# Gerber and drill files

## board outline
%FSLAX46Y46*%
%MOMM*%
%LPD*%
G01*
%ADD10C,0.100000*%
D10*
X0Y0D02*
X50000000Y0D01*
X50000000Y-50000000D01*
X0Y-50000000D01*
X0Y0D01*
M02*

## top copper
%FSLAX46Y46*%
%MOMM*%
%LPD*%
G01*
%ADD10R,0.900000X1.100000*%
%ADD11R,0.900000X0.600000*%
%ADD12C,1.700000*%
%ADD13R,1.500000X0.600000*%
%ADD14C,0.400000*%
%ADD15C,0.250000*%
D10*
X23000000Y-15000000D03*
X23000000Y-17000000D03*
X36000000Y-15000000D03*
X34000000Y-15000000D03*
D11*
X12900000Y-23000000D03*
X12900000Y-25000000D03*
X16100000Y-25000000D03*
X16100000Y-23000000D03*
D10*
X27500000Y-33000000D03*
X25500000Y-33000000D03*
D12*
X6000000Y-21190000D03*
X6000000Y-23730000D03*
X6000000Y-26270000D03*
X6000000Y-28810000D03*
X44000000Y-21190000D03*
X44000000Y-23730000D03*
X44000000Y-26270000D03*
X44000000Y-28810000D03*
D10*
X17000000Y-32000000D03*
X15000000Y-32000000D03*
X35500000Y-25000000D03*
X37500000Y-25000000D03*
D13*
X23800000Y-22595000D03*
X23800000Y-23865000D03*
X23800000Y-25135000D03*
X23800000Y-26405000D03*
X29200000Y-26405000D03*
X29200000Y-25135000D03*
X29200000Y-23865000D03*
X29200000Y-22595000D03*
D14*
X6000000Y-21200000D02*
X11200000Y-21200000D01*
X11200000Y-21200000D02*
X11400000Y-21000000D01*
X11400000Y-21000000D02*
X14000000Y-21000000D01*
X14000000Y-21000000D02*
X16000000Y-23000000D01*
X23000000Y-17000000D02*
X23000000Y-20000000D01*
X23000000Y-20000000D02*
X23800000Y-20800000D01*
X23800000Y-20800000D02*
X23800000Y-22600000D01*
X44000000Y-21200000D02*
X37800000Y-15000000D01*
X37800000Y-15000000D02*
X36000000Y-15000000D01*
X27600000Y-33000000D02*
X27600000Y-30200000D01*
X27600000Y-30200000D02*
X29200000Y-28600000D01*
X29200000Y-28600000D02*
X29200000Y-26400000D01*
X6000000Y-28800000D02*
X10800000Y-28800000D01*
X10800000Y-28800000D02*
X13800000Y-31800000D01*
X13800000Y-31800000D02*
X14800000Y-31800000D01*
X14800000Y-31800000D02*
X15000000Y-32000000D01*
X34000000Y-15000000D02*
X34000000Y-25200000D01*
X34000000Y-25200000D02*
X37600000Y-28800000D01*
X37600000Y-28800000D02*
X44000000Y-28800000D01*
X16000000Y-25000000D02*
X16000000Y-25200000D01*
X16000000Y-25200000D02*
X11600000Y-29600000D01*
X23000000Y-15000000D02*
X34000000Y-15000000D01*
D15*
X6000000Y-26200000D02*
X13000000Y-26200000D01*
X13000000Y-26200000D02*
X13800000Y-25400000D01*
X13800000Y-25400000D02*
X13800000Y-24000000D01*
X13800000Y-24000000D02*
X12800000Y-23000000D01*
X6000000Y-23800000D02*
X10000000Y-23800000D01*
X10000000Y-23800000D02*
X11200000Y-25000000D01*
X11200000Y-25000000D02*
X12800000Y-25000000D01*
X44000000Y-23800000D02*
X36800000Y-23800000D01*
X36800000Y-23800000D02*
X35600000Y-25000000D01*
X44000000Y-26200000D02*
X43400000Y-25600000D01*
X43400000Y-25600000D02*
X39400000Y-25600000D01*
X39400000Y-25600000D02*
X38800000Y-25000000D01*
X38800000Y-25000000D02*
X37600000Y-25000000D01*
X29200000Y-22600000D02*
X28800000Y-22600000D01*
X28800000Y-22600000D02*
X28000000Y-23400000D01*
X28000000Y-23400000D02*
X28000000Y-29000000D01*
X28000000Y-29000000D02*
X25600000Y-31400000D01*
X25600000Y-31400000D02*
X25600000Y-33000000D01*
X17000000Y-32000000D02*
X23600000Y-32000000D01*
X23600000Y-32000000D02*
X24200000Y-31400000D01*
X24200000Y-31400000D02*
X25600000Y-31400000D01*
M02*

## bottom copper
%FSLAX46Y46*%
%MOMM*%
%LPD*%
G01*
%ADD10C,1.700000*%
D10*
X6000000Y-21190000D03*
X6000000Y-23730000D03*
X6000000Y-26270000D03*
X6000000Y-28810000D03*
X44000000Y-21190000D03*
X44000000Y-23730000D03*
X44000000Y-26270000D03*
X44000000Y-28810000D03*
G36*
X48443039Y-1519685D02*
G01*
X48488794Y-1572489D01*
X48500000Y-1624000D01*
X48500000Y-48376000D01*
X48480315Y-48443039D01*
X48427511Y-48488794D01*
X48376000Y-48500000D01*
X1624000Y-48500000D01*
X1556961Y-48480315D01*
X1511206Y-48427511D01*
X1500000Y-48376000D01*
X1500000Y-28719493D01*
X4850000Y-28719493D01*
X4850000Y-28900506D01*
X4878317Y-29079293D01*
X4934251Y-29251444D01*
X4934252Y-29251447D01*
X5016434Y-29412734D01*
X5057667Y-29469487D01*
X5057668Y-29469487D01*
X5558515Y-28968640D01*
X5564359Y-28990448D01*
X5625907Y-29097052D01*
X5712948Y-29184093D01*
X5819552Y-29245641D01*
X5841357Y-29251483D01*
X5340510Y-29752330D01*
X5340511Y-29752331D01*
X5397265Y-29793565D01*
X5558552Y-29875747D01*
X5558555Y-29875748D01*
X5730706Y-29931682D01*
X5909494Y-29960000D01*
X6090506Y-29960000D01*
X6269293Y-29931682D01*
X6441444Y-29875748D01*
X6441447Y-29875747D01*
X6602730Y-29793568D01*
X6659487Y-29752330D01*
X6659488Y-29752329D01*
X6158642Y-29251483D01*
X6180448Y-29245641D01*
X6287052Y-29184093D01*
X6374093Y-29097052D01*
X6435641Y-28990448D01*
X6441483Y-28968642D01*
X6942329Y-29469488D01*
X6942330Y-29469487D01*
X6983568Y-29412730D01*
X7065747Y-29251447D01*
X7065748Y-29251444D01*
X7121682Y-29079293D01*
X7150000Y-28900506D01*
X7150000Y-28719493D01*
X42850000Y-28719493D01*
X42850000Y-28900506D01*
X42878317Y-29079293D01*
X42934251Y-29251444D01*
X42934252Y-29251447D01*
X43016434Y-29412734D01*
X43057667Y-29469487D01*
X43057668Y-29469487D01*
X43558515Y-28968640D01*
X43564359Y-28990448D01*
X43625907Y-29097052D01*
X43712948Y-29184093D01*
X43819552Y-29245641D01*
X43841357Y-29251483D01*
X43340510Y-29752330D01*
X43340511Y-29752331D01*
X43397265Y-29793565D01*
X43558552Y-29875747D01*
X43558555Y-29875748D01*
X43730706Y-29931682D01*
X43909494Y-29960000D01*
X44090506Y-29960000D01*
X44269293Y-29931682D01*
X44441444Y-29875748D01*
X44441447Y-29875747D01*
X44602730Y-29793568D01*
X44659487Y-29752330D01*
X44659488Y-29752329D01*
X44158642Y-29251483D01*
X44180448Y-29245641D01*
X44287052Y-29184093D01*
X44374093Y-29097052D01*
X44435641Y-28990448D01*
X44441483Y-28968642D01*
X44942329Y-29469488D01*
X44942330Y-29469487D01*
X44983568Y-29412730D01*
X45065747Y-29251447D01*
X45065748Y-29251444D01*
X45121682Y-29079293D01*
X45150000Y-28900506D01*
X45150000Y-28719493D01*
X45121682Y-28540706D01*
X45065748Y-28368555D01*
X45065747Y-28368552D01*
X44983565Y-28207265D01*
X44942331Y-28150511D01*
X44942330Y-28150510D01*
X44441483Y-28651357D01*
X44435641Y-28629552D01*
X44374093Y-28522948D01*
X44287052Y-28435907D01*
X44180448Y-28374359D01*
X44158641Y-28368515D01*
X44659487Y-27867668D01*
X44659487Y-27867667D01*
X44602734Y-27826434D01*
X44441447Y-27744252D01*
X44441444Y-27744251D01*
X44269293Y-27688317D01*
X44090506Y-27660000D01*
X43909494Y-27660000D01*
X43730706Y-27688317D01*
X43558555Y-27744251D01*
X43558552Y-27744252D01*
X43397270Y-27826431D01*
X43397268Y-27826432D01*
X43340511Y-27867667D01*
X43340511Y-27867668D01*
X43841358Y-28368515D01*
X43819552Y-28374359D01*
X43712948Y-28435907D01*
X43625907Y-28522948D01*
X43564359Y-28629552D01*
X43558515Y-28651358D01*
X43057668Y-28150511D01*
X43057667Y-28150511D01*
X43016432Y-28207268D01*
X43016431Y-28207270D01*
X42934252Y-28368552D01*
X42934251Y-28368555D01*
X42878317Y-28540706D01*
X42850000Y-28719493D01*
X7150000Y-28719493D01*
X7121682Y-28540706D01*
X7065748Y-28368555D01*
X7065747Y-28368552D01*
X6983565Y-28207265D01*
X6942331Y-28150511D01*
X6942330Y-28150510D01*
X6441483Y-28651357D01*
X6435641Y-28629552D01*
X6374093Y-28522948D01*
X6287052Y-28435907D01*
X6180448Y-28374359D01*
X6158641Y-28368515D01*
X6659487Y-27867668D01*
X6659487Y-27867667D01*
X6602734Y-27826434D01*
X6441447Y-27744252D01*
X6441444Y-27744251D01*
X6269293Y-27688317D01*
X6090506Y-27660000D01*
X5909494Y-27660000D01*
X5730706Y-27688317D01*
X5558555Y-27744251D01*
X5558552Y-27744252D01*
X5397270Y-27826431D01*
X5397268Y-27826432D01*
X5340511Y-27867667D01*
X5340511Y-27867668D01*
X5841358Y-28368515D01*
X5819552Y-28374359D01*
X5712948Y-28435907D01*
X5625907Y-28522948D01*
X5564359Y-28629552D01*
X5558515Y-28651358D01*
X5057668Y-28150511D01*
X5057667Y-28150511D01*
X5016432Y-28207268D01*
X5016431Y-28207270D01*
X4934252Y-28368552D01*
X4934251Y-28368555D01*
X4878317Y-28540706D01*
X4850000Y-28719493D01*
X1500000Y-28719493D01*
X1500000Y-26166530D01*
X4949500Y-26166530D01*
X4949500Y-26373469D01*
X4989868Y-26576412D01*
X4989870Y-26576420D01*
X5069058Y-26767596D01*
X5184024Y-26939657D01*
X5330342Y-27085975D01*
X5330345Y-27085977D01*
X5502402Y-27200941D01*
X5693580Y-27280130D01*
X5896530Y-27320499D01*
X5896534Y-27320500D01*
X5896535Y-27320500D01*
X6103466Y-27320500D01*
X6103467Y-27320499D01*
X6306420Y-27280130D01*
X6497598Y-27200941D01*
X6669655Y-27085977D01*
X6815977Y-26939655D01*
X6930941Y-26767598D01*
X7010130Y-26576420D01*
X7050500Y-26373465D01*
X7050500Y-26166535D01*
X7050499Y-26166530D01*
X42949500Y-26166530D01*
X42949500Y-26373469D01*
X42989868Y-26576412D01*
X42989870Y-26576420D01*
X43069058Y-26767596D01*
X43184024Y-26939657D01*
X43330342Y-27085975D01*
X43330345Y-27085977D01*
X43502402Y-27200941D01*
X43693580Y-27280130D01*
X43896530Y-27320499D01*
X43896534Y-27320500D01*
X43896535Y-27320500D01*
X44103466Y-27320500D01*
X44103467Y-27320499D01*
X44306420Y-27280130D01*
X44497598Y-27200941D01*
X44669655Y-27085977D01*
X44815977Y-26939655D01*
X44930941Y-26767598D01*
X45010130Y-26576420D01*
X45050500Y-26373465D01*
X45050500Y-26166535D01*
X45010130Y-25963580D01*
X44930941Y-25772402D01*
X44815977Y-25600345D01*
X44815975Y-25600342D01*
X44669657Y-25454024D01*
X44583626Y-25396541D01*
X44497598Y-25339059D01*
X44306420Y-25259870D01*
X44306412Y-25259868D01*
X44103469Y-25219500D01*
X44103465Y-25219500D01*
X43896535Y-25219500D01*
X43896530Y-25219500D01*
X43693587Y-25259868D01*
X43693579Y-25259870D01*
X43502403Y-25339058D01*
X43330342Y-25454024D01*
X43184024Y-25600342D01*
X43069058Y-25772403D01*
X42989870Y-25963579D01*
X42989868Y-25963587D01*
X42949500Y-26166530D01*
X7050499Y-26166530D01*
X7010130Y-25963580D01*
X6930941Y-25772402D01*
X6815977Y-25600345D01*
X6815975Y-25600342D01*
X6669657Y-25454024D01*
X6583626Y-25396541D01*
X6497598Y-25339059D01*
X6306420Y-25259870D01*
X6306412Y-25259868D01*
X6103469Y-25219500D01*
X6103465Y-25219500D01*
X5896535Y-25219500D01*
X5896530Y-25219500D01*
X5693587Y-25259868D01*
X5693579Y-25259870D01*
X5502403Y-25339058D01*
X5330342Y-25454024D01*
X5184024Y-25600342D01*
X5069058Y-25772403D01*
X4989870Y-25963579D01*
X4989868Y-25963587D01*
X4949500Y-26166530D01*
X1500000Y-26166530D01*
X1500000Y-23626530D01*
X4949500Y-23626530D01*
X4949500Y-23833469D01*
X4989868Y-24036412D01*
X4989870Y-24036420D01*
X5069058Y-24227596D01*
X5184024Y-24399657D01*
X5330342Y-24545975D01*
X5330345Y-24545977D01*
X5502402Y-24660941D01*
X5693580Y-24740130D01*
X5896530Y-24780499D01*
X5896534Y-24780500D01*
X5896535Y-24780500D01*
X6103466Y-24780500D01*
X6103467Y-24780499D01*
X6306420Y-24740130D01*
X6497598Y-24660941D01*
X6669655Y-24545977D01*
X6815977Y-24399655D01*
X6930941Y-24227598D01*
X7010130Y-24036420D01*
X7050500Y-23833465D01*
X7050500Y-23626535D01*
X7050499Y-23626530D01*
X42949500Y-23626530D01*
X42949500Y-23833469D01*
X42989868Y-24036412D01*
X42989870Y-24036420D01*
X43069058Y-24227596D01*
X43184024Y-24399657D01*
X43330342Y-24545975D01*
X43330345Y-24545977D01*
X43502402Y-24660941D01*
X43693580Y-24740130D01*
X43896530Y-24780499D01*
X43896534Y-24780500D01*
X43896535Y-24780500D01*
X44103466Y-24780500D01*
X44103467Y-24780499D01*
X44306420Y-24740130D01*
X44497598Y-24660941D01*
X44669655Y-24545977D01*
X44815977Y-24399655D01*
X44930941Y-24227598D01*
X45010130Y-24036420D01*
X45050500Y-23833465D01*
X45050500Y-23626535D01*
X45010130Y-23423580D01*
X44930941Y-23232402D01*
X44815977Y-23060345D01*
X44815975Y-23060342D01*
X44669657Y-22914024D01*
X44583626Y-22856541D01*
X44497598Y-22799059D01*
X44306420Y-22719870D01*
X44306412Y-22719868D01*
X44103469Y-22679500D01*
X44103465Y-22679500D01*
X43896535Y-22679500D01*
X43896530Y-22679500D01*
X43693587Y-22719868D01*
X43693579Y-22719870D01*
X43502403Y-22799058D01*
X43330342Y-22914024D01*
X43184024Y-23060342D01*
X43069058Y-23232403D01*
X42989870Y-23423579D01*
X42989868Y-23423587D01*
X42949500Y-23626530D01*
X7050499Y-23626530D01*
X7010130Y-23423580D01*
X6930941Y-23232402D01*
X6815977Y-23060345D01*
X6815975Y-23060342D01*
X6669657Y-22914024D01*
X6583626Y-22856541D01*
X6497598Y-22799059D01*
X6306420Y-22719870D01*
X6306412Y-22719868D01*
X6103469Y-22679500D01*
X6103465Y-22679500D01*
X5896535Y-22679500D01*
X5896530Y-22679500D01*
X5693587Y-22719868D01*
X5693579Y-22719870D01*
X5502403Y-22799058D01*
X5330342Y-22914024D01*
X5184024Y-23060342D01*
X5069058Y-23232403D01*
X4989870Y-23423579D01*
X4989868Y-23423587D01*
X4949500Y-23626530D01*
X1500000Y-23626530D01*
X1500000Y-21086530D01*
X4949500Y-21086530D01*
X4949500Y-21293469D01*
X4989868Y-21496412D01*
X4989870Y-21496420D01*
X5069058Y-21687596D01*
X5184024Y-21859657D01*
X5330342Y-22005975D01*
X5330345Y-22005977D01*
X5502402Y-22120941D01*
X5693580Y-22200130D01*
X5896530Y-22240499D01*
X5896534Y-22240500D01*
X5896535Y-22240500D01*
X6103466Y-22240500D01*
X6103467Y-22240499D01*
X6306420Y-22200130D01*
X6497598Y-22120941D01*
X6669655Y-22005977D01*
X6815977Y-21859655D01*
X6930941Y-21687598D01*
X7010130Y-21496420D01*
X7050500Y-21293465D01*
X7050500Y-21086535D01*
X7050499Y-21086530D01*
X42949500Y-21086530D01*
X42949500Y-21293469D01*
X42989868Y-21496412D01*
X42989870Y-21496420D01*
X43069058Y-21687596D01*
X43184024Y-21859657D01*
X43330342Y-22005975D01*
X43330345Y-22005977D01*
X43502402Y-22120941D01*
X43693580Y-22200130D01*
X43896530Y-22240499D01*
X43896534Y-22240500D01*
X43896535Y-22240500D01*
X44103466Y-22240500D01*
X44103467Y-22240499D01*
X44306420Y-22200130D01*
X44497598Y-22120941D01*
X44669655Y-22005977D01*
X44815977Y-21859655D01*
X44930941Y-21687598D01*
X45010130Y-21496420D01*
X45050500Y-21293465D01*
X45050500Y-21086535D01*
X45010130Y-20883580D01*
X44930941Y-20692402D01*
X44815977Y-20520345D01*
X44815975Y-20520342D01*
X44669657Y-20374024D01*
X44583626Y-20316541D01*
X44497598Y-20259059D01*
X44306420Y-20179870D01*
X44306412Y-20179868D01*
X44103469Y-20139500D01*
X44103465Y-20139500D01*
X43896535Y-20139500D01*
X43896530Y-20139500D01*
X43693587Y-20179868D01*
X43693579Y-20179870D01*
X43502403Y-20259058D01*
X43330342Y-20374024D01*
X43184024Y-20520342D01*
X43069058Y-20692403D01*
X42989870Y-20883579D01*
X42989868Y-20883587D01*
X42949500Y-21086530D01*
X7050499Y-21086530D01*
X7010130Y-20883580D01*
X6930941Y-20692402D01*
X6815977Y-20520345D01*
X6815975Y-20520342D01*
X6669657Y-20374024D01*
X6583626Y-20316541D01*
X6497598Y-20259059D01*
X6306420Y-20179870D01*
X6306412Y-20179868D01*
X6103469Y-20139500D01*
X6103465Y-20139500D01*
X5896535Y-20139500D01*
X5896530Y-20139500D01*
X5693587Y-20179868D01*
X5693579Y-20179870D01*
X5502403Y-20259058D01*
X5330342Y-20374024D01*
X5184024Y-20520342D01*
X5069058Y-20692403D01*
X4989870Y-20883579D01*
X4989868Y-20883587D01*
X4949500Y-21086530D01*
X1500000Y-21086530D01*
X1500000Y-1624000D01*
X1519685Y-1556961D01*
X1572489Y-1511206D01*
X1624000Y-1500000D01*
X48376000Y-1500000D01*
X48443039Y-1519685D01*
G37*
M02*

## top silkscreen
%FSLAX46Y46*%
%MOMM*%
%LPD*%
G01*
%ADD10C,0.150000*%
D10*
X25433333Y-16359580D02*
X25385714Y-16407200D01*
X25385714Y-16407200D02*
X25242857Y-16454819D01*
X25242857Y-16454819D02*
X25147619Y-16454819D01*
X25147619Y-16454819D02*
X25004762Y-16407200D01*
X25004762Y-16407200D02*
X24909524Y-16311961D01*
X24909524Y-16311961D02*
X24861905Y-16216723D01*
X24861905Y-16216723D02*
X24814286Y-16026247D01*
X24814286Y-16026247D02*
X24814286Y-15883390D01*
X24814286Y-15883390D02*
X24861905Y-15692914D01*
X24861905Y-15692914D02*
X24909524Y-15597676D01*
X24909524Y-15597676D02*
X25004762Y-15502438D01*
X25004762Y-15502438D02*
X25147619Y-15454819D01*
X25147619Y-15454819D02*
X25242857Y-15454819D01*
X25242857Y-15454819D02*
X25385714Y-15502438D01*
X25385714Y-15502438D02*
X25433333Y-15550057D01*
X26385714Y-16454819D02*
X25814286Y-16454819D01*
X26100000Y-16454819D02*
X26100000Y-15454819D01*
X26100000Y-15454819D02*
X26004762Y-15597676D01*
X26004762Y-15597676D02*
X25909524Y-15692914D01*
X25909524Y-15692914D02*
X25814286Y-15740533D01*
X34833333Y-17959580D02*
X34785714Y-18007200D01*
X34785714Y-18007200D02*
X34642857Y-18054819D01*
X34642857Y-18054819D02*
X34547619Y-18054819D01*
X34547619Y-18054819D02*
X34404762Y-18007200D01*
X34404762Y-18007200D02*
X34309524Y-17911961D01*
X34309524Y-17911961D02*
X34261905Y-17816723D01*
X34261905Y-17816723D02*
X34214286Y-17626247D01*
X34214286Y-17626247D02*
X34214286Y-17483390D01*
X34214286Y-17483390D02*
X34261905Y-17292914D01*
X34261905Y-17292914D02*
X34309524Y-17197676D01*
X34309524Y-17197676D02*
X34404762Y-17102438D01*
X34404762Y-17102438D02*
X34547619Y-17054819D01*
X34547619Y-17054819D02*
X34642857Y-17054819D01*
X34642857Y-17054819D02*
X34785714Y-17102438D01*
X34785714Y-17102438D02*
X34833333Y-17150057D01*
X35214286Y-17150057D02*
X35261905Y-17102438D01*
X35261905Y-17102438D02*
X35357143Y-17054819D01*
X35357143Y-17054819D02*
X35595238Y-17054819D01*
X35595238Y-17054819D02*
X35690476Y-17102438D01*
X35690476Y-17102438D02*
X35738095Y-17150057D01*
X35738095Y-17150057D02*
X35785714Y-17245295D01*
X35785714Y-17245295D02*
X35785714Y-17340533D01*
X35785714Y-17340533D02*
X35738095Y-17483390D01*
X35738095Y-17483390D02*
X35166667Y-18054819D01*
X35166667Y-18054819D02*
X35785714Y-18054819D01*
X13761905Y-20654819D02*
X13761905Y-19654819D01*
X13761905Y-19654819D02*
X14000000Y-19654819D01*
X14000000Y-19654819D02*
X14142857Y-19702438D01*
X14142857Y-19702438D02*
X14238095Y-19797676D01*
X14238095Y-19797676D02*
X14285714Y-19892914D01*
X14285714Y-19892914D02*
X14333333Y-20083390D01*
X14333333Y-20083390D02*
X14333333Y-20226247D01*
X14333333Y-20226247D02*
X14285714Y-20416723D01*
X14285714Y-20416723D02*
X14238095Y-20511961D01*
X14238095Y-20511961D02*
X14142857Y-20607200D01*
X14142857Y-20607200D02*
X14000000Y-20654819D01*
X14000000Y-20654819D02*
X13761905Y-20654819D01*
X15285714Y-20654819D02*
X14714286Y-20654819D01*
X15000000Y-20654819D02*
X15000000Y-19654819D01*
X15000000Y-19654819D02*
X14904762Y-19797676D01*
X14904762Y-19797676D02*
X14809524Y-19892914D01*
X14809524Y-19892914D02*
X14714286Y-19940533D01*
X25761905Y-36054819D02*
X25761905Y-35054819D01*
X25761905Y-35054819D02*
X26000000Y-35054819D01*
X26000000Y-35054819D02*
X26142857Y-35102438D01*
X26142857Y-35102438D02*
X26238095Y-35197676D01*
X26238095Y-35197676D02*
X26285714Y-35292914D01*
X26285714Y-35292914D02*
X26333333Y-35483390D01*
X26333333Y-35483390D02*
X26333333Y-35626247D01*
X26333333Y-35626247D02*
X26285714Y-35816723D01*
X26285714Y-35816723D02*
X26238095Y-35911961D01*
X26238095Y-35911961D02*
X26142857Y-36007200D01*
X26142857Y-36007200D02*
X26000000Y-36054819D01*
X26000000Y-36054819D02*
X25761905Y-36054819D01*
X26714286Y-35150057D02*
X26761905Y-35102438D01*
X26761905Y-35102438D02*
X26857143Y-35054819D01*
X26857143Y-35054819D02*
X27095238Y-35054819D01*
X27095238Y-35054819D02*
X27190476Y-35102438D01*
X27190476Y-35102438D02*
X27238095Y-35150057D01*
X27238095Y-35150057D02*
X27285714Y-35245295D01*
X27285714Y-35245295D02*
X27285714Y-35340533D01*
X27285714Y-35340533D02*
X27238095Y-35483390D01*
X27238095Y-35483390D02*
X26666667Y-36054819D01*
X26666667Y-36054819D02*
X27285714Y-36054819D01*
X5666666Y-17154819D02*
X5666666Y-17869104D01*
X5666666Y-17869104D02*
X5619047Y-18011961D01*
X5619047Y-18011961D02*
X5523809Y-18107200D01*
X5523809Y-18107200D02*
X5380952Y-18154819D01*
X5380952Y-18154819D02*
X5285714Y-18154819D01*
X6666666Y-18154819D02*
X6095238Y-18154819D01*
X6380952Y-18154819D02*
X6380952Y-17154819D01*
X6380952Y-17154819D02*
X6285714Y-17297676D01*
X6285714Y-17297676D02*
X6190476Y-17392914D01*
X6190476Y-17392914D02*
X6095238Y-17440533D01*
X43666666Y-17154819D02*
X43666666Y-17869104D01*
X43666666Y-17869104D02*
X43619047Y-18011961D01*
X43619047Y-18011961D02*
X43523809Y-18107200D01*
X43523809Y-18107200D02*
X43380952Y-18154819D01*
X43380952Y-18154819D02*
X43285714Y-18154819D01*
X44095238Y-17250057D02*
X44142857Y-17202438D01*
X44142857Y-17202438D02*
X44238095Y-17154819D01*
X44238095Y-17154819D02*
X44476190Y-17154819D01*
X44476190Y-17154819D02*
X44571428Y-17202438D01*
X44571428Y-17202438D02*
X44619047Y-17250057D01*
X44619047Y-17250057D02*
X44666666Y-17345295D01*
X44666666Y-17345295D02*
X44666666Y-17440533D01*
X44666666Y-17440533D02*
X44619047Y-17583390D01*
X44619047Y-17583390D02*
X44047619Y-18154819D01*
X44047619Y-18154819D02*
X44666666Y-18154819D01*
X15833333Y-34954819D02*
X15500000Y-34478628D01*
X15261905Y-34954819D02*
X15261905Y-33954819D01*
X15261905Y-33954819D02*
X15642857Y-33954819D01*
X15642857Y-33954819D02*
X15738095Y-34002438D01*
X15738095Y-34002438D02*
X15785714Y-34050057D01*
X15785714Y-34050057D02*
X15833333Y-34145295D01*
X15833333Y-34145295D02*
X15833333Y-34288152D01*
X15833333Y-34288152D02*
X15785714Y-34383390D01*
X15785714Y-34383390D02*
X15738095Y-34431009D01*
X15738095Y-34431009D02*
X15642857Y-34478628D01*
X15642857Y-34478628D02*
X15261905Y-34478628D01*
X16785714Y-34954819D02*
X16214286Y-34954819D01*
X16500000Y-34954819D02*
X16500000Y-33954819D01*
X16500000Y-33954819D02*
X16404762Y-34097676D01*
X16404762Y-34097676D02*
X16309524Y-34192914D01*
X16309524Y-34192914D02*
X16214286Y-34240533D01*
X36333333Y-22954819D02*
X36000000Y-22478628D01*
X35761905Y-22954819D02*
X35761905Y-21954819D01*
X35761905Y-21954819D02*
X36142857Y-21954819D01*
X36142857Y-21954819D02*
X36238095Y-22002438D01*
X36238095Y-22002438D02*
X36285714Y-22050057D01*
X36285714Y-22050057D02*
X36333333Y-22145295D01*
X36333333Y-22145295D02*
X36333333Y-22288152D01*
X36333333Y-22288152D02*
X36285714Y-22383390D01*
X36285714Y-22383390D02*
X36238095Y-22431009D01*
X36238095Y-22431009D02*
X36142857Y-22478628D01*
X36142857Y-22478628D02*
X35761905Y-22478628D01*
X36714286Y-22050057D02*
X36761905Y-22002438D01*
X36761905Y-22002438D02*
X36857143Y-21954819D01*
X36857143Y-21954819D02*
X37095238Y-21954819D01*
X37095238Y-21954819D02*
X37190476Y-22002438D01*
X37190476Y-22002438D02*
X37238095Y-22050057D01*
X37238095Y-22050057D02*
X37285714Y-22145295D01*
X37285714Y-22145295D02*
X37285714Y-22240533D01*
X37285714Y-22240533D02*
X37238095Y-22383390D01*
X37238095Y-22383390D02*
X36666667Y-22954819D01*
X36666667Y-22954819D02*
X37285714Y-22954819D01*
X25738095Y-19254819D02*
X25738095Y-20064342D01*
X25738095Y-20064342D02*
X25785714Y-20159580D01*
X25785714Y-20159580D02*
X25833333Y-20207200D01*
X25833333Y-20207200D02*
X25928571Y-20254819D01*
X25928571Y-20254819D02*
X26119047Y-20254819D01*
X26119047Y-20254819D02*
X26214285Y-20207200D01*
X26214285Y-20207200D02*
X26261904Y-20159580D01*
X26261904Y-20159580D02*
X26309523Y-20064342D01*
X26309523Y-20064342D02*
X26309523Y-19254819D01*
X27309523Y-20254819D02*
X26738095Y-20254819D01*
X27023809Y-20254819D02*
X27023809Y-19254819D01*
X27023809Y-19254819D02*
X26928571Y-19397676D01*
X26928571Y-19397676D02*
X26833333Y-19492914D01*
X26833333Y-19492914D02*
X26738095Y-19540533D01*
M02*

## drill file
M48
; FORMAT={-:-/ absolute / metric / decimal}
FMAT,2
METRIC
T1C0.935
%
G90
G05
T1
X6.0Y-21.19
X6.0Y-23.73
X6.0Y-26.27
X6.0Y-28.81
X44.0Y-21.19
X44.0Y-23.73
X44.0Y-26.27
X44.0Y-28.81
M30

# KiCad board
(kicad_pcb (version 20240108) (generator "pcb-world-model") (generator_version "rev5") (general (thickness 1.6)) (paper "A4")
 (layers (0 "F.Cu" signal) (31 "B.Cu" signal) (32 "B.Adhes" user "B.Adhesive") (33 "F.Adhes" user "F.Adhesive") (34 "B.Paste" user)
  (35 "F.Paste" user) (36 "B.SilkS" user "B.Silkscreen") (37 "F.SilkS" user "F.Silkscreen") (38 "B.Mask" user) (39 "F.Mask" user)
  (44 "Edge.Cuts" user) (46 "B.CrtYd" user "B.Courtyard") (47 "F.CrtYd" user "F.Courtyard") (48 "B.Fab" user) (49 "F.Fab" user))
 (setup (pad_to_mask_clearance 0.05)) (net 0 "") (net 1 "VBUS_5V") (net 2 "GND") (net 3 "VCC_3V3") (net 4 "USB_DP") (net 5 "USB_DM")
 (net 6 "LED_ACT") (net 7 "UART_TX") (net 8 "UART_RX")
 (gr_rect (start 0.0 0.0) (end 50.0000 50.0000) (stroke (width 0.1) (type default)) (fill none) (layer "Edge.Cuts"))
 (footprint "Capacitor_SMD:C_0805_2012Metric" (layer "F.Cu") (at 23.0000 16.0000 270)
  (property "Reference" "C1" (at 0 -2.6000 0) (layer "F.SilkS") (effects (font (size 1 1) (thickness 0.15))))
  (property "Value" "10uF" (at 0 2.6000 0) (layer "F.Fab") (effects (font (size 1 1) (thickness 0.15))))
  (pad "1" smd rect (at -1.0000 0.0000) (size 0.9000 1.1000) (layers "F.Cu" "F.Paste" "F.Mask") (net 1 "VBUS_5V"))
  (pad "2" smd rect (at 1.0000 0.0000) (size 0.9000 1.1000) (layers "F.Cu" "F.Paste" "F.Mask") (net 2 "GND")))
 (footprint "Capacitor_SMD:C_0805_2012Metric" (layer "F.Cu") (at 35.0000 15.0000 180)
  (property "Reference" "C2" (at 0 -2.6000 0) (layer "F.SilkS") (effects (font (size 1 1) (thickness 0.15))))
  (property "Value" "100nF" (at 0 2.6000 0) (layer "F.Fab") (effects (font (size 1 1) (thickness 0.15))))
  (pad "1" smd rect (at -1.0000 0.0000) (size 0.9000 1.1000) (layers "F.Cu" "F.Paste" "F.Mask") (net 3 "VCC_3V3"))
  (pad "2" smd rect (at 1.0000 0.0000) (size 0.9000 1.1000) (layers "F.Cu" "F.Paste" "F.Mask") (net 2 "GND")))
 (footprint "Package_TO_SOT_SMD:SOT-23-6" (layer "F.Cu") (at 14.5000 24.0000 0)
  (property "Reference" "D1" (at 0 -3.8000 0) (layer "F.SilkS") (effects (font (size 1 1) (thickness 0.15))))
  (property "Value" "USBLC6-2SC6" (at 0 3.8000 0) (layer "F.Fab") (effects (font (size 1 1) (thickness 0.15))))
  (pad "1" smd rect (at -1.6000 -1.0000) (size 0.9000 0.6000) (layers "F.Cu" "F.Paste" "F.Mask") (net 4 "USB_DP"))
  (pad "2" smd rect (at -1.6000 1.0000) (size 0.9000 0.6000) (layers "F.Cu" "F.Paste" "F.Mask") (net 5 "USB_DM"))
  (pad "3" smd rect (at 1.6000 1.0000) (size 0.9000 0.6000) (layers "F.Cu" "F.Paste" "F.Mask") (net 2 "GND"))
  (pad "4" smd rect (at 1.6000 -1.0000) (size 0.9000 0.6000) (layers "F.Cu" "F.Paste" "F.Mask") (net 1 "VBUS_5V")))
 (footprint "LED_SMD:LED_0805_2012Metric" (layer "F.Cu") (at 26.5000 33.0000 180)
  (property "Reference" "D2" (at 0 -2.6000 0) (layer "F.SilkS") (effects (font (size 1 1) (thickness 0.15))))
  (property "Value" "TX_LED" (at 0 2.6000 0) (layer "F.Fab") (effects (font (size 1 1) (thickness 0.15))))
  (pad "1" smd rect (at -1.0000 0.0000) (size 0.9000 1.1000) (layers "F.Cu" "F.Paste" "F.Mask") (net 3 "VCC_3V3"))
  (pad "2" smd rect (at 1.0000 0.0000) (size 0.9000 1.1000) (layers "F.Cu" "F.Paste" "F.Mask") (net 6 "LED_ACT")))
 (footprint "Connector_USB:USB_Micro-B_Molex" (layer "F.Cu") (at 6.0000 25.0000 0) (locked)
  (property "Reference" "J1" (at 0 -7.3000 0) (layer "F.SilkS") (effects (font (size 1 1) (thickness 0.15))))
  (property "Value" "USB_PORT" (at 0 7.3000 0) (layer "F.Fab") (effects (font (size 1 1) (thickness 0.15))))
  (pad "1" thru_hole circle (at 0.0000 -3.8100) (size 1.7000 1.7000) (drill 0.9350) (layers "*.Cu" "*.Mask") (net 1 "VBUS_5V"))
  (pad "2" thru_hole circle (at 0.0000 -1.2700) (size 1.7000 1.7000) (drill 0.9350) (layers "*.Cu" "*.Mask") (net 5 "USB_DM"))
  (pad "3" thru_hole circle (at 0.0000 1.2700) (size 1.7000 1.7000) (drill 0.9350) (layers "*.Cu" "*.Mask") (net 4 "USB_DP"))
  (pad "4" thru_hole circle (at 0.0000 3.8100) (size 1.7000 1.7000) (drill 0.9350) (layers "*.Cu" "*.Mask") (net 2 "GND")))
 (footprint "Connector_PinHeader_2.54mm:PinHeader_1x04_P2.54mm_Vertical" (layer "F.Cu") (at 44.0000 25.0000 0) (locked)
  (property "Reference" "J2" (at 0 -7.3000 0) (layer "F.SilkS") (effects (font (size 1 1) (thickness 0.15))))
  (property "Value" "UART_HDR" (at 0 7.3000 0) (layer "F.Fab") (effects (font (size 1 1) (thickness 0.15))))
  (pad "1" thru_hole circle (at 0.0000 -3.8100) (size 1.7000 1.7000) (drill 0.9350) (layers "*.Cu" "*.Mask") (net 3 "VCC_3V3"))
  (pad "2" thru_hole circle (at 0.0000 -1.2700) (size 1.7000 1.7000) (drill 0.9350) (layers "*.Cu" "*.Mask") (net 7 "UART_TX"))
  (pad "3" thru_hole circle (at 0.0000 1.2700) (size 1.7000 1.7000) (drill 0.9350) (layers "*.Cu" "*.Mask") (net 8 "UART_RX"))
  (pad "4" thru_hole circle (at 0.0000 3.8100) (size 1.7000 1.7000) (drill 0.9350) (layers "*.Cu" "*.Mask") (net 2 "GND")))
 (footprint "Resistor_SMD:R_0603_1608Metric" (layer "F.Cu") (at 16.0000 32.0000 180)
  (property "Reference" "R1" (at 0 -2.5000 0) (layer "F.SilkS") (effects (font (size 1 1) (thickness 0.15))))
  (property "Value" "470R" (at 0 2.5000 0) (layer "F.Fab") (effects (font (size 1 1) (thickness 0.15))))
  (pad "1" smd rect (at -1.0000 0.0000) (size 0.9000 1.1000) (layers "F.Cu" "F.Paste" "F.Mask") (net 6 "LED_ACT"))
  (pad "2" smd rect (at 1.0000 0.0000) (size 0.9000 1.1000) (layers "F.Cu" "F.Paste" "F.Mask") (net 2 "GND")))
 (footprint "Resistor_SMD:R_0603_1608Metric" (layer "F.Cu") (at 36.5000 25.0000 0)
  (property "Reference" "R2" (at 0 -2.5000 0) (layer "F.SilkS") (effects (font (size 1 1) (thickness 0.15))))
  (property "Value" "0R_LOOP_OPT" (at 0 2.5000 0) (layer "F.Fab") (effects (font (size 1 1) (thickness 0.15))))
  (pad "1" smd rect (at -1.0000 0.0000) (size 0.9000 1.1000) (layers "F.Cu" "F.Paste" "F.Mask") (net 7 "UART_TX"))
  (pad "2" smd rect (at 1.0000 0.0000) (size 0.9000 1.1000) (layers "F.Cu" "F.Paste" "F.Mask") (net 8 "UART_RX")))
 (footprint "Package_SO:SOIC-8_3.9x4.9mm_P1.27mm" (layer "F.Cu") (at 26.5000 24.5000 0)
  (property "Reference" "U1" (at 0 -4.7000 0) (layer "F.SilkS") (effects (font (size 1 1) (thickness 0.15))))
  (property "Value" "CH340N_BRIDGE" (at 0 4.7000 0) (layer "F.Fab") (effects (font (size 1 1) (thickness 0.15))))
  (pad "1" smd rect (at -2.7000 -1.9050) (size 1.5000 0.6000) (layers "F.Cu" "F.Paste" "F.Mask") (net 1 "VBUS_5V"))
  (pad "2" smd rect (at -2.7000 -0.6350) (size 1.5000 0.6000) (layers "F.Cu" "F.Paste" "F.Mask") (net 4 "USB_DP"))
  (pad "3" smd rect (at -2.7000 0.6350) (size 1.5000 0.6000) (layers "F.Cu" "F.Paste" "F.Mask") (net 5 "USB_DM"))
  (pad "4" smd rect (at -2.7000 1.9050) (size 1.5000 0.6000) (layers "F.Cu" "F.Paste" "F.Mask") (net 2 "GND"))
  (pad "5" smd rect (at 2.7000 1.9050) (size 1.5000 0.6000) (layers "F.Cu" "F.Paste" "F.Mask") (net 3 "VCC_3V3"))
  (pad "6" smd rect (at 2.7000 0.6350) (size 1.5000 0.6000) (layers "F.Cu" "F.Paste" "F.Mask") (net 7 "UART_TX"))
  (pad "7" smd rect (at 2.7000 -0.6350) (size 1.5000 0.6000) (layers "F.Cu" "F.Paste" "F.Mask") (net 8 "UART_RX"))
  (pad "8" smd rect (at 2.7000 -1.9050) (size 1.5000 0.6000) (layers "F.Cu" "F.Paste" "F.Mask") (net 6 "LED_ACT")))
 (segment (start 6.0000 21.2000) (end 11.2000 21.2000) (width 0.4000) (layer "F.Cu") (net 1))
 (segment (start 11.2000 21.2000) (end 11.4000 21.0000) (width 0.4000) (layer "F.Cu") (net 1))
 (segment (start 11.4000 21.0000) (end 14.0000 21.0000) (width 0.4000) (layer "F.Cu") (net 1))
 (segment (start 14.0000 21.0000) (end 16.0000 23.0000) (width 0.4000) (layer "F.Cu") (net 1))
 (segment (start 23.0000 17.0000) (end 23.0000 20.0000) (width 0.4000) (layer "F.Cu") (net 1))
 (segment (start 23.0000 20.0000) (end 23.8000 20.8000) (width 0.4000) (layer "F.Cu") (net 1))
 (segment (start 23.8000 20.8000) (end 23.8000 22.6000) (width 0.4000) (layer "F.Cu") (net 1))
 (segment (start 44.0000 21.2000) (end 37.8000 15.0000) (width 0.4000) (layer "F.Cu") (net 3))
 (segment (start 37.8000 15.0000) (end 36.0000 15.0000) (width 0.4000) (layer "F.Cu") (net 3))
 (segment (start 27.6000 33.0000) (end 27.6000 30.2000) (width 0.4000) (layer "F.Cu") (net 3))
 (segment (start 27.6000 30.2000) (end 29.2000 28.6000) (width 0.4000) (layer "F.Cu") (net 3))
 (segment (start 29.2000 28.6000) (end 29.2000 26.4000) (width 0.4000) (layer "F.Cu") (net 3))
 (segment (start 6.0000 28.8000) (end 10.8000 28.8000) (width 0.4000) (layer "F.Cu") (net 2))
 (segment (start 10.8000 28.8000) (end 13.8000 31.8000) (width 0.4000) (layer "F.Cu") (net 2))
 (segment (start 13.8000 31.8000) (end 14.8000 31.8000) (width 0.4000) (layer "F.Cu") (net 2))
 (segment (start 14.8000 31.8000) (end 15.0000 32.0000) (width 0.4000) (layer "F.Cu") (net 2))
 (segment (start 34.0000 15.0000) (end 34.0000 25.2000) (width 0.4000) (layer "F.Cu") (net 2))
 (segment (start 34.0000 25.2000) (end 37.6000 28.8000) (width 0.4000) (layer "F.Cu") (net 2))
 (segment (start 37.6000 28.8000) (end 44.0000 28.8000) (width 0.4000) (layer "F.Cu") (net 2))
 (segment (start 16.0000 25.0000) (end 16.0000 25.2000) (width 0.4000) (layer "F.Cu") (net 2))
 (segment (start 16.0000 25.2000) (end 11.6000 29.6000) (width 0.4000) (layer "F.Cu") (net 2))
 (segment (start 23.0000 15.0000) (end 34.0000 15.0000) (width 0.4000) (layer "F.Cu") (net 2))
 (segment (start 6.0000 26.2000) (end 13.0000 26.2000) (width 0.2500) (layer "F.Cu") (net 4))
 (segment (start 13.0000 26.2000) (end 13.8000 25.4000) (width 0.2500) (layer "F.Cu") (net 4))
 (segment (start 13.8000 25.4000) (end 13.8000 24.0000) (width 0.2500) (layer "F.Cu") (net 4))
 (segment (start 13.8000 24.0000) (end 12.8000 23.0000) (width 0.2500) (layer "F.Cu") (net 4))
 (segment (start 6.0000 23.8000) (end 10.0000 23.8000) (width 0.2500) (layer "F.Cu") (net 5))
 (segment (start 10.0000 23.8000) (end 11.2000 25.0000) (width 0.2500) (layer "F.Cu") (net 5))
 (segment (start 11.2000 25.0000) (end 12.8000 25.0000) (width 0.2500) (layer "F.Cu") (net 5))
 (segment (start 44.0000 23.8000) (end 36.8000 23.8000) (width 0.2500) (layer "F.Cu") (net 7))
 (segment (start 36.8000 23.8000) (end 35.6000 25.0000) (width 0.2500) (layer "F.Cu") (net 7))
 (segment (start 44.0000 26.2000) (end 43.4000 25.6000) (width 0.2500) (layer "F.Cu") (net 8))
 (segment (start 43.4000 25.6000) (end 39.4000 25.6000) (width 0.2500) (layer "F.Cu") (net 8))
 (segment (start 39.4000 25.6000) (end 38.8000 25.0000) (width 0.2500) (layer "F.Cu") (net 8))
 (segment (start 38.8000 25.0000) (end 37.6000 25.0000) (width 0.2500) (layer "F.Cu") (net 8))
 (segment (start 29.2000 22.6000) (end 28.8000 22.6000) (width 0.2500) (layer "F.Cu") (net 6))
 (segment (start 28.8000 22.6000) (end 28.0000 23.4000) (width 0.2500) (layer "F.Cu") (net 6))
 (segment (start 28.0000 23.4000) (end 28.0000 29.0000) (width 0.2500) (layer "F.Cu") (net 6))
 (segment (start 28.0000 29.0000) (end 25.6000 31.4000) (width 0.2500) (layer "F.Cu") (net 6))
 (segment (start 25.6000 31.4000) (end 25.6000 33.0000) (width 0.2500) (layer "F.Cu") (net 6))
 (segment (start 17.0000 32.0000) (end 23.6000 32.0000) (width 0.2500) (layer "F.Cu") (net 6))
 (segment (start 23.6000 32.0000) (end 24.2000 31.4000) (width 0.2500) (layer "F.Cu") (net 6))
 (segment (start 24.2000 31.4000) (end 25.6000 31.4000) (width 0.2500) (layer "F.Cu") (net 6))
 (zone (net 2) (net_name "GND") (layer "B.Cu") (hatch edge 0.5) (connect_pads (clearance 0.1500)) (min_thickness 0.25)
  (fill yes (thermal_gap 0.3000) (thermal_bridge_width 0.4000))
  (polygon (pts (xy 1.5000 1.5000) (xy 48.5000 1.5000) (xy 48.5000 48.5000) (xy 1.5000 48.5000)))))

